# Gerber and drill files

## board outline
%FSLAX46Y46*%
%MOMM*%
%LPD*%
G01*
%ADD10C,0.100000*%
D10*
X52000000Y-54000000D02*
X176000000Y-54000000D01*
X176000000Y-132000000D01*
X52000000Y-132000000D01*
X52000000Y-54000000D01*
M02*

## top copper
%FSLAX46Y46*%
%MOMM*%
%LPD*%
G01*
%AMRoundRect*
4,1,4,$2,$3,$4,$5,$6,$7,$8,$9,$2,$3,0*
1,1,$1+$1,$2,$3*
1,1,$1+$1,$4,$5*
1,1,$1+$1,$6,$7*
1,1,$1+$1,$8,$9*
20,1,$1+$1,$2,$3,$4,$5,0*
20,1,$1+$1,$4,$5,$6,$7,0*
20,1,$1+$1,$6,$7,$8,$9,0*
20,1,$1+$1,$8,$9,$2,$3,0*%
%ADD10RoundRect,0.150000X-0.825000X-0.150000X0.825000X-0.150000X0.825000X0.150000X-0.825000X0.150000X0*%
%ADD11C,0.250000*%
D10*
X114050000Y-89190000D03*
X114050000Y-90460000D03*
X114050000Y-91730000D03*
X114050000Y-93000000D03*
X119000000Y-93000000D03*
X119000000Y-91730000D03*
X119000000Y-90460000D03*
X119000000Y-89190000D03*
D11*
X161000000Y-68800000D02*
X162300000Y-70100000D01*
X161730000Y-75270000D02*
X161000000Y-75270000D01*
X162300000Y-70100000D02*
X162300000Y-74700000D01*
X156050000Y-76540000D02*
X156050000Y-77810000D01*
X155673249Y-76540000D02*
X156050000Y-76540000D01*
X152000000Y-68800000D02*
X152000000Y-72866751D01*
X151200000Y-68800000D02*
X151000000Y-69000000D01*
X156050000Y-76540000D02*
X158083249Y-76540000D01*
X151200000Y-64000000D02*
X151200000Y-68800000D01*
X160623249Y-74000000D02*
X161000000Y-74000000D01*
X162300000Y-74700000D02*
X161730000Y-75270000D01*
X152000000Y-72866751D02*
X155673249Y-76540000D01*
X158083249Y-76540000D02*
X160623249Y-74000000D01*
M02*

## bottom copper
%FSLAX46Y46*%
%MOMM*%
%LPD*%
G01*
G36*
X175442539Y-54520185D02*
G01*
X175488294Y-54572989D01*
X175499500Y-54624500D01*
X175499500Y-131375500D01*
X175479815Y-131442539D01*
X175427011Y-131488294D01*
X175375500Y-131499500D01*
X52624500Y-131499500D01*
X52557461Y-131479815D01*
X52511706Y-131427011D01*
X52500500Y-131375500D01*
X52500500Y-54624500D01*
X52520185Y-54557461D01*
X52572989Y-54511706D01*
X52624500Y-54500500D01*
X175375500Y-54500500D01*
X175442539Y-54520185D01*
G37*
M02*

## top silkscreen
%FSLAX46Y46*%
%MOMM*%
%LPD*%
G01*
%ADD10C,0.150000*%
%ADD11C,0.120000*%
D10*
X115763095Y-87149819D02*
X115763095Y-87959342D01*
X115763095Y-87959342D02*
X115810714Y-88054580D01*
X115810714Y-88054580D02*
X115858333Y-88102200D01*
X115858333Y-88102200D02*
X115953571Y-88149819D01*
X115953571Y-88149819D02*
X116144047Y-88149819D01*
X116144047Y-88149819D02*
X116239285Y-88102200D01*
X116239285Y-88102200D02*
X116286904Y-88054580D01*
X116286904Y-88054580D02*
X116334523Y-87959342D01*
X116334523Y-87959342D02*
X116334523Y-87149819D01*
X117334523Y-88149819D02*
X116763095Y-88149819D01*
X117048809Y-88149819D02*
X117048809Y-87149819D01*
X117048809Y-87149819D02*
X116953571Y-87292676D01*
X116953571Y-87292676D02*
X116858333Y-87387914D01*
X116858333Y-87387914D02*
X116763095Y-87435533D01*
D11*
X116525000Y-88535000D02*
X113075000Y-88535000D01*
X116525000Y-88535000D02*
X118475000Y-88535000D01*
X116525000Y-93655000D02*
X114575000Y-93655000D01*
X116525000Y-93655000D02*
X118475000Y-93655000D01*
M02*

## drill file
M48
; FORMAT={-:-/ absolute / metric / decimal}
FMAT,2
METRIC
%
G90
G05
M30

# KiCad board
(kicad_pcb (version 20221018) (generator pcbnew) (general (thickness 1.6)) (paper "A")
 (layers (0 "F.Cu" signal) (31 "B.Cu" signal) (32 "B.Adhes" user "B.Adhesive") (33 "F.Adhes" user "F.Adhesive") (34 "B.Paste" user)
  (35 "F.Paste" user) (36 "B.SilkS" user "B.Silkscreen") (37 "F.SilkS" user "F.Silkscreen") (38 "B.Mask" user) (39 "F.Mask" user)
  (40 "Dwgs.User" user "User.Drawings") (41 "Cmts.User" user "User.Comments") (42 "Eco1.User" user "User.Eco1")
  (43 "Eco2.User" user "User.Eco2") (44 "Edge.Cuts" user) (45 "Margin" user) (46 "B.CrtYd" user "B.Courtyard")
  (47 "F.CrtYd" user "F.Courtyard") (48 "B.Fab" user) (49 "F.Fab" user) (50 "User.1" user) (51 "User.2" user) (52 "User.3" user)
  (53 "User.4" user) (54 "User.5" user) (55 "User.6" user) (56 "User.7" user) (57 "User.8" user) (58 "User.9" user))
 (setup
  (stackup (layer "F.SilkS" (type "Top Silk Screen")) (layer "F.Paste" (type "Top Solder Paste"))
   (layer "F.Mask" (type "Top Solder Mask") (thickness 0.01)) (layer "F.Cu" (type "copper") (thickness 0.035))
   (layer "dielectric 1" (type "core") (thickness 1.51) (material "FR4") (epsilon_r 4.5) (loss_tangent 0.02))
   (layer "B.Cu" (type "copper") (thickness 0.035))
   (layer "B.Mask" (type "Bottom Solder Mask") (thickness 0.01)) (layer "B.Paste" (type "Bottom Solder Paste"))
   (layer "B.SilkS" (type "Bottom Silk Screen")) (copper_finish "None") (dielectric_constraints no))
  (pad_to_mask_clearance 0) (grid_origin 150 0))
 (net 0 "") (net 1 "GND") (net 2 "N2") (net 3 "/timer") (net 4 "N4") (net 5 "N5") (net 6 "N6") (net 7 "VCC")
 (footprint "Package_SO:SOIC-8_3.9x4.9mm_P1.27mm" (layer "F.Cu") (at 116.525 91.095)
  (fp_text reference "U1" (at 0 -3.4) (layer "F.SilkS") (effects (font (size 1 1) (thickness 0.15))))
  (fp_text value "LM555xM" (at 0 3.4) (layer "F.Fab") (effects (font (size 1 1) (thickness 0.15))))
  (fp_line (start 0 -2.56) (end -3.45 -2.56) (stroke (width 0.12) (type solid)) (layer "F.SilkS"))
  (fp_line (start 0 -2.56) (end 1.95 -2.56) (stroke (width 0.12) (type solid)) (layer "F.SilkS"))
  (fp_line (start 0 2.56) (end -1.95 2.56) (stroke (width 0.12) (type solid)) (layer "F.SilkS"))
  (fp_line (start 0 2.56) (end 1.95 2.56) (stroke (width 0.12) (type solid)) (layer "F.SilkS"))
  (pad "1" smd roundrect (at -2.475 -1.905) (size 1.95 0.6) (layers "F.Cu" "F.Paste" "F.Mask") (roundrect_rratio 0.25) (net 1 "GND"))
  (pad "2" smd roundrect (at -2.475 -0.635) (size 1.95 0.6) (layers "F.Cu" "F.Paste" "F.Mask") (roundrect_rratio 0.25) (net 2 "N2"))
  (pad "3" smd roundrect (at -2.475 0.635) (size 1.95 0.6) (layers "F.Cu" "F.Paste" "F.Mask") (roundrect_rratio 0.25) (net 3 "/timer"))
  (pad "4" smd roundrect (at -2.475 1.905) (size 1.95 0.6) (layers "F.Cu" "F.Paste" "F.Mask") (roundrect_rratio 0.25) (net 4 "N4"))
  (pad "5" smd roundrect (at 2.475 1.905) (size 1.95 0.6) (layers "F.Cu" "F.Paste" "F.Mask") (roundrect_rratio 0.25) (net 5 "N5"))
  (pad "6" smd roundrect (at 2.475 0.635) (size 1.95 0.6) (layers "F.Cu" "F.Paste" "F.Mask") (roundrect_rratio 0.25) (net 2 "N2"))
  (pad "7" smd roundrect (at 2.475 -0.635) (size 1.95 0.6) (layers "F.Cu" "F.Paste" "F.Mask") (roundrect_rratio 0.25) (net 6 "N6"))
  (pad "8" smd roundrect (at 2.475 -1.905) (size 1.95 0.6) (layers "F.Cu" "F.Paste" "F.Mask") (roundrect_rratio 0.25) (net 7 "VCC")))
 (gr_rect (start 52 54) (end 176 132) (stroke (width 0.1) (type default)) (fill none) (layer "Edge.Cuts"))
 (segment (start 161 68.8) (end 162.3 70.1) (width 0.25) (layer "F.Cu") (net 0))
 (segment (start 161.73 75.27) (end 161 75.27) (width 0.25) (layer "F.Cu") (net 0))
 (segment (start 162.3 70.1) (end 162.3 74.7) (width 0.25) (layer "F.Cu") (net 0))
 (segment (start 156.05 76.54) (end 156.05 77.81) (width 0.25) (layer "F.Cu") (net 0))
 (segment (start 155.673249 76.54) (end 156.05 76.54) (width 0.25) (layer "F.Cu") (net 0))
 (segment (start 152 68.8) (end 152 72.866751) (width 0.25) (layer "F.Cu") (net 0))
 (segment (start 151.2 68.8) (end 151 69) (width 0.25) (layer "F.Cu") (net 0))
 (segment (start 156.05 76.54) (end 158.083249 76.54) (width 0.25) (layer "F.Cu") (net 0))
 (segment (start 151.2 64) (end 151.2 68.8) (width 0.25) (layer "F.Cu") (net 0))
 (segment (start 160.623249 74) (end 161 74) (width 0.25) (layer "F.Cu") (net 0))
 (segment (start 162.3 74.7) (end 161.73 75.27) (width 0.25) (layer "F.Cu") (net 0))
 (segment (start 152 72.866751) (end 155.673249 76.54) (width 0.25) (layer "F.Cu") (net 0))
 (segment (start 158.083249 76.54) (end 160.623249 74) (width 0.25) (layer "F.Cu") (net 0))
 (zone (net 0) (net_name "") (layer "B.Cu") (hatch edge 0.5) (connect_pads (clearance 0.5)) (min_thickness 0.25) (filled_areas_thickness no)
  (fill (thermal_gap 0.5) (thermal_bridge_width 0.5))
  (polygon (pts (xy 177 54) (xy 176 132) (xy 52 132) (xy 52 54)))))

